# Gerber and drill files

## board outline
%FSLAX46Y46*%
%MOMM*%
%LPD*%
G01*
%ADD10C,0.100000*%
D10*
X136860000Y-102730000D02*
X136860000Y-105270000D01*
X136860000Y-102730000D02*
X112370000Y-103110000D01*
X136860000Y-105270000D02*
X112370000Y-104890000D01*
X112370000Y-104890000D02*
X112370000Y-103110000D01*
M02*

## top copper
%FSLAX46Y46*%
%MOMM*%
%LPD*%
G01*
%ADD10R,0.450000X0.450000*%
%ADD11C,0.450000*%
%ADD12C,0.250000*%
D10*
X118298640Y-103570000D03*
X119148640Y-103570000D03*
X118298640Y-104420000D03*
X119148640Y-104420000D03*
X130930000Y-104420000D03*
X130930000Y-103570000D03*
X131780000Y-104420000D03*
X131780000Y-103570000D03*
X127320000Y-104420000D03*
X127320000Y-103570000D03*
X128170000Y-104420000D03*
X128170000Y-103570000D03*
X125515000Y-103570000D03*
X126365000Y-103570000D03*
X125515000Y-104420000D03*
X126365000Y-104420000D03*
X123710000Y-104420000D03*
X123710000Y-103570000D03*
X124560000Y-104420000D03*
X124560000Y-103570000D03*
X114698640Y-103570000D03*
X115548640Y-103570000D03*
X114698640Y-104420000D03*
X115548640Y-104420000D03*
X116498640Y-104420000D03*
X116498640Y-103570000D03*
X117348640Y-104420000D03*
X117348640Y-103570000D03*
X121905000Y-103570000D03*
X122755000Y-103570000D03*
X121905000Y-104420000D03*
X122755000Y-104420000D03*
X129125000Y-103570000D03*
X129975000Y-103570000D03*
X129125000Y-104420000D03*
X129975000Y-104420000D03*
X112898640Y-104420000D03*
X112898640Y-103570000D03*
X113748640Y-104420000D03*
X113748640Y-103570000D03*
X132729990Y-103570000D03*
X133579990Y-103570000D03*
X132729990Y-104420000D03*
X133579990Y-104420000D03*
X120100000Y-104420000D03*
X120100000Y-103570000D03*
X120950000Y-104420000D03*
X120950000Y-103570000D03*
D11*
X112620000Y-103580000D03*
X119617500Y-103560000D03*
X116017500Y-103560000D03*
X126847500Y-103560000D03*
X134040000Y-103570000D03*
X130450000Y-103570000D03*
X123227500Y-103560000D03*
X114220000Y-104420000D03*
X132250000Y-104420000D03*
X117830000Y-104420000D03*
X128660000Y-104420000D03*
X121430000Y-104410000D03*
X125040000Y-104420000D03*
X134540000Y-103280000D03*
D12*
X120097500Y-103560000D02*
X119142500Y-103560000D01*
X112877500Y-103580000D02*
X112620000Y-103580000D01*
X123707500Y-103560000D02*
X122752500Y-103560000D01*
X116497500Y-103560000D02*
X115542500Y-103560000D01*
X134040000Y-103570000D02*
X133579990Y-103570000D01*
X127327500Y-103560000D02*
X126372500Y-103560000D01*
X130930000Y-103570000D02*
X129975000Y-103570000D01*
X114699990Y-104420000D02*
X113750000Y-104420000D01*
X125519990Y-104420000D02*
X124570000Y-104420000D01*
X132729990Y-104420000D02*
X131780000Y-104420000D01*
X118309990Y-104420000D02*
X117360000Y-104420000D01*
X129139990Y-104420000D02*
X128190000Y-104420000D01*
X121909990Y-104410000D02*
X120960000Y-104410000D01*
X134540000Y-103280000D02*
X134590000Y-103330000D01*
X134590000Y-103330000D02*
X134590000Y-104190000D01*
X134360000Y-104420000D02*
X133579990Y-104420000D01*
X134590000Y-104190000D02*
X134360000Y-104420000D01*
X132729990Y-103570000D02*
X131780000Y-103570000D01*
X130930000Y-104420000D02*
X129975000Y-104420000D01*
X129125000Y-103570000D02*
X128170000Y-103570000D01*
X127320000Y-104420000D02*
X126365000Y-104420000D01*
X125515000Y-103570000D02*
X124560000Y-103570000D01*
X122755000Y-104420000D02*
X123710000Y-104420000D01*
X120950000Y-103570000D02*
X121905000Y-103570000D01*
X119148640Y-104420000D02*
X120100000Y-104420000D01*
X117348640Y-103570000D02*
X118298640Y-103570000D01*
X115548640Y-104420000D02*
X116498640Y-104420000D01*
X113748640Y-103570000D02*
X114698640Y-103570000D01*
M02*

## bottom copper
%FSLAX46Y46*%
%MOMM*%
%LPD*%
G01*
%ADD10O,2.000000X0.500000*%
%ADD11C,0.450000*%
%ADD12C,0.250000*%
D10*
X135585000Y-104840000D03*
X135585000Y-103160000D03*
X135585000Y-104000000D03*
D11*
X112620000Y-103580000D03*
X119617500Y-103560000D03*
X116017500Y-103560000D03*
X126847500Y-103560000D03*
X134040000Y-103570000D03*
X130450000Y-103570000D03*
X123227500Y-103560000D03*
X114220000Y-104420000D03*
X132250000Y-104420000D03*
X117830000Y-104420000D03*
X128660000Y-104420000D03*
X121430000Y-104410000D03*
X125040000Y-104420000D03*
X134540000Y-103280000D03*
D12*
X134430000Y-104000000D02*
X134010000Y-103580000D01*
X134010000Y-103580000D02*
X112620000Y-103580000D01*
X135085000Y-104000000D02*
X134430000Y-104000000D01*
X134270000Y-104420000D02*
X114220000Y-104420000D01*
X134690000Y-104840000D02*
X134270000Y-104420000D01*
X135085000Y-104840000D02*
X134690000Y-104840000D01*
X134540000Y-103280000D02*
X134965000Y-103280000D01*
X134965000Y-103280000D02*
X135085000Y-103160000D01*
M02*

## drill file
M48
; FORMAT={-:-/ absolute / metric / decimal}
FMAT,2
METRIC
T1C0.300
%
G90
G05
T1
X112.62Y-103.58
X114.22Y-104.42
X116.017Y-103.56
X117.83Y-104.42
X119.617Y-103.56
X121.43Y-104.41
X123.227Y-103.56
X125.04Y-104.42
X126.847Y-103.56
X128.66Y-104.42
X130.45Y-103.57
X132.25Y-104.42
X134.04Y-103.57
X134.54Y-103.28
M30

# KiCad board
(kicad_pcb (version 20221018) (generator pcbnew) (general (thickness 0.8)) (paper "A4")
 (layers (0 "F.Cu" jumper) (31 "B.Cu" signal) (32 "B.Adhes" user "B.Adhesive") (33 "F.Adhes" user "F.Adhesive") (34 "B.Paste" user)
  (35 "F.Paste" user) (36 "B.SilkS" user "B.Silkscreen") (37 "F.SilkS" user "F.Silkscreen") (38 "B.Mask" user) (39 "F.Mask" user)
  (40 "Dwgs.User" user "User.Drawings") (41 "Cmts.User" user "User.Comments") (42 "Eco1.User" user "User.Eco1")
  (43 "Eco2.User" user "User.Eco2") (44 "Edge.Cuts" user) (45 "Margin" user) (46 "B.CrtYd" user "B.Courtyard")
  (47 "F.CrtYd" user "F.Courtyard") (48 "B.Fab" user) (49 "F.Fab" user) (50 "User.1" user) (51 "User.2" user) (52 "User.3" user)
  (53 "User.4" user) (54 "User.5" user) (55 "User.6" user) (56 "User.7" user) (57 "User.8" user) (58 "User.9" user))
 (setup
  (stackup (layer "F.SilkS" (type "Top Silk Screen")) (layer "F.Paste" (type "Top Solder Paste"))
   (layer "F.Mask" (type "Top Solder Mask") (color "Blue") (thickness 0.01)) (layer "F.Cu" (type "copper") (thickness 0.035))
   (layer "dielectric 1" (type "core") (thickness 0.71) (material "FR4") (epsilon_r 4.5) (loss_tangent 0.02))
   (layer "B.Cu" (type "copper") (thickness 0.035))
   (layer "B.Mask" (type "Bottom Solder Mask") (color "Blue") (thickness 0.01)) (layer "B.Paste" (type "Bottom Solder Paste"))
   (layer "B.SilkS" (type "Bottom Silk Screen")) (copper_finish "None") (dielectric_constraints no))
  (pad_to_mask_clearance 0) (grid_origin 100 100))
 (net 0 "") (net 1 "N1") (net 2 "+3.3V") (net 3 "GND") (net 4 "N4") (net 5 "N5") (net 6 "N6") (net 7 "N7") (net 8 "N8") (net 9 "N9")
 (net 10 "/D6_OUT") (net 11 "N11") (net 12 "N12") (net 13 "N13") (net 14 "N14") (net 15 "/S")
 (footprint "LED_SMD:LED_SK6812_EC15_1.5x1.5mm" (layer "F.Cu") (at 118.72364 103.995)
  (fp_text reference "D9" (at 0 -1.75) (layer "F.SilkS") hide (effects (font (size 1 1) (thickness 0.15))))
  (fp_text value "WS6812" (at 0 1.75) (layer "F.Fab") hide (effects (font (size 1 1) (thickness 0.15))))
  (pad "1" smd rect (at -0.425 -0.425) (size 0.45 0.45) (layers "F.Cu" "F.Paste" "F.Mask") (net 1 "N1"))
  (pad "2" smd rect (at 0.425 -0.425) (size 0.45 0.45) (layers "F.Cu" "F.Paste" "F.Mask") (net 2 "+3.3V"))
  (pad "3" smd rect (at -0.425 0.425) (size 0.45 0.45) (layers "F.Cu" "F.Paste" "F.Mask") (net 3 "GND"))
  (pad "4" smd rect (at 0.425 0.425) (size 0.45 0.45) (layers "F.Cu" "F.Paste" "F.Mask") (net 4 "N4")))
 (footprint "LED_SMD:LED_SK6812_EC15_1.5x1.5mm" (layer "F.Cu") (at 131.355 103.995 90)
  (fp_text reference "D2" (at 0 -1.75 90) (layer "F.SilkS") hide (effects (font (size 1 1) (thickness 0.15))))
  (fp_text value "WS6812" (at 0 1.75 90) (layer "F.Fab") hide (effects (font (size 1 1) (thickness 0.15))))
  (pad "1" smd rect (at -0.425 -0.425 90) (size 0.45 0.45) (layers "F.Cu" "F.Paste" "F.Mask") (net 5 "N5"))
  (pad "2" smd rect (at 0.425 -0.425 90) (size 0.45 0.45) (layers "F.Cu" "F.Paste" "F.Mask") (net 2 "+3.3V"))
  (pad "3" smd rect (at -0.425 0.425 90) (size 0.45 0.45) (layers "F.Cu" "F.Paste" "F.Mask") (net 3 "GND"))
  (pad "4" smd rect (at 0.425 0.425 90) (size 0.45 0.45) (layers "F.Cu" "F.Paste" "F.Mask") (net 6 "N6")))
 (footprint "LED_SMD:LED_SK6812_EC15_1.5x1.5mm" (layer "F.Cu") (at 127.745 103.995 90)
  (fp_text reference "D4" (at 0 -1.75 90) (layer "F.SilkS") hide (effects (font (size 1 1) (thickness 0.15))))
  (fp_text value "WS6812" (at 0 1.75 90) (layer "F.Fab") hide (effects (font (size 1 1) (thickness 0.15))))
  (pad "1" smd rect (at -0.425 -0.425 90) (size 0.45 0.45) (layers "F.Cu" "F.Paste" "F.Mask") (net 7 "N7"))
  (pad "2" smd rect (at 0.425 -0.425 90) (size 0.45 0.45) (layers "F.Cu" "F.Paste" "F.Mask") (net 2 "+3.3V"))
  (pad "3" smd rect (at -0.425 0.425 90) (size 0.45 0.45) (layers "F.Cu" "F.Paste" "F.Mask") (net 3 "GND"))
  (pad "4" smd rect (at 0.425 0.425 90) (size 0.45 0.45) (layers "F.Cu" "F.Paste" "F.Mask") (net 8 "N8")))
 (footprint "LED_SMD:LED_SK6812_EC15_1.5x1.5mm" (layer "F.Cu") (at 125.94 103.995)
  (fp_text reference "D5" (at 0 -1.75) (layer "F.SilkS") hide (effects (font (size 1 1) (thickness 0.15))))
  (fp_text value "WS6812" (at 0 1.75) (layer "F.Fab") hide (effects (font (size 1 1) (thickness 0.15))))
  (pad "1" smd rect (at -0.425 -0.425) (size 0.45 0.45) (layers "F.Cu" "F.Paste" "F.Mask") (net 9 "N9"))
  (pad "2" smd rect (at 0.425 -0.425) (size 0.45 0.45) (layers "F.Cu" "F.Paste" "F.Mask") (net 2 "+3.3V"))
  (pad "3" smd rect (at -0.425 0.425) (size 0.45 0.45) (layers "F.Cu" "F.Paste" "F.Mask") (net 3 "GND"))
  (pad "4" smd rect (at 0.425 0.425) (size 0.45 0.45) (layers "F.Cu" "F.Paste" "F.Mask") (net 7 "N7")))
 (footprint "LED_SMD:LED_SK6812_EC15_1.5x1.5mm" (layer "F.Cu") (at 124.135 103.995 90)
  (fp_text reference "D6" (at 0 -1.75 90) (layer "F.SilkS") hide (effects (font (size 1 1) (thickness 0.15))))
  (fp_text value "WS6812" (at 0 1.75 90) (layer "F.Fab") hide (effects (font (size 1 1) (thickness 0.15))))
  (pad "1" smd rect (at -0.425 -0.425 90) (size 0.45 0.45) (layers "F.Cu" "F.Paste" "F.Mask") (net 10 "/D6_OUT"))
  (pad "2" smd rect (at 0.425 -0.425 90) (size 0.45 0.45) (layers "F.Cu" "F.Paste" "F.Mask") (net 2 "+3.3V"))
  (pad "3" smd rect (at -0.425 0.425 90) (size 0.45 0.45) (layers "F.Cu" "F.Paste" "F.Mask") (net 3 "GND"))
  (pad "4" smd rect (at 0.425 0.425 90) (size 0.45 0.45) (layers "F.Cu" "F.Paste" "F.Mask") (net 9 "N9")))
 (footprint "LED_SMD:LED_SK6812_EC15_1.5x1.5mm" (layer "F.Cu") (at 115.12364 103.995)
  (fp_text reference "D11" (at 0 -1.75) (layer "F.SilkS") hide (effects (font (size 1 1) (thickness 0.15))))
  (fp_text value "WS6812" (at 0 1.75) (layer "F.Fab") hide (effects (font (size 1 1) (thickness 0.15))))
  (pad "1" smd rect (at -0.425 -0.425) (size 0.45 0.45) (layers "F.Cu" "F.Paste" "F.Mask") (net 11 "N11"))
  (pad "2" smd rect (at 0.425 -0.425) (size 0.45 0.45) (layers "F.Cu" "F.Paste" "F.Mask") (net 2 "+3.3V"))
  (pad "3" smd rect (at -0.425 0.425) (size 0.45 0.45) (layers "F.Cu" "F.Paste" "F.Mask") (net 3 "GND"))
  (pad "4" smd rect (at 0.425 0.425) (size 0.45 0.45) (layers "F.Cu" "F.Paste" "F.Mask") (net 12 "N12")))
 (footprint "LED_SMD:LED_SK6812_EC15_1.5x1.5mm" (layer "F.Cu") (at 116.92364 103.995 90)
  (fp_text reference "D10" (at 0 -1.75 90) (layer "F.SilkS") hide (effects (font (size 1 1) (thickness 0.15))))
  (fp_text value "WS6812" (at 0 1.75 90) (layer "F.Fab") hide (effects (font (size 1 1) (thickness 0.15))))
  (pad "1" smd rect (at -0.425 -0.425 90) (size 0.45 0.45) (layers "F.Cu" "F.Paste" "F.Mask") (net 12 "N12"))
  (pad "2" smd rect (at 0.425 -0.425 90) (size 0.45 0.45) (layers "F.Cu" "F.Paste" "F.Mask") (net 2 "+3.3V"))
  (pad "3" smd rect (at -0.425 0.425 90) (size 0.45 0.45) (layers "F.Cu" "F.Paste" "F.Mask") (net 3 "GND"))
  (pad "4" smd rect (at 0.425 0.425 90) (size 0.45 0.45) (layers "F.Cu" "F.Paste" "F.Mask") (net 1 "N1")))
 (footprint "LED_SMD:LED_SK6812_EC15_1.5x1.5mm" (layer "F.Cu") (at 122.33 103.995)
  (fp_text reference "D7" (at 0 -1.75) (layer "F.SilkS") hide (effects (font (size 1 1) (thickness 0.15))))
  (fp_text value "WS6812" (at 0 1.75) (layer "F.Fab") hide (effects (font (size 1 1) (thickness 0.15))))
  (pad "1" smd rect (at -0.425 -0.425) (size 0.45 0.45) (layers "F.Cu" "F.Paste" "F.Mask") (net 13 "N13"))
  (pad "2" smd rect (at 0.425 -0.425) (size 0.45 0.45) (layers "F.Cu" "F.Paste" "F.Mask") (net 2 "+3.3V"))
  (pad "3" smd rect (at -0.425 0.425) (size 0.45 0.45) (layers "F.Cu" "F.Paste" "F.Mask") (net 3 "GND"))
  (pad "4" smd rect (at 0.425 0.425) (size 0.45 0.45) (layers "F.Cu" "F.Paste" "F.Mask") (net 10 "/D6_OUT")))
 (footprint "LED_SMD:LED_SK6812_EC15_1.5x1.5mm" (layer "F.Cu") (at 129.55 103.995)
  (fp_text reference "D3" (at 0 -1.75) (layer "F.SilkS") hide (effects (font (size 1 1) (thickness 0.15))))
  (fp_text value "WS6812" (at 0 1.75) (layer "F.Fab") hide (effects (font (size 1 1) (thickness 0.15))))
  (pad "1" smd rect (at -0.425 -0.425) (size 0.45 0.45) (layers "F.Cu" "F.Paste" "F.Mask") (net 8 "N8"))
  (pad "2" smd rect (at 0.425 -0.425) (size 0.45 0.45) (layers "F.Cu" "F.Paste" "F.Mask") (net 2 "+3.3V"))
  (pad "3" smd rect (at -0.425 0.425) (size 0.45 0.45) (layers "F.Cu" "F.Paste" "F.Mask") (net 3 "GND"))
  (pad "4" smd rect (at 0.425 0.425) (size 0.45 0.45) (layers "F.Cu" "F.Paste" "F.Mask") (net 5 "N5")))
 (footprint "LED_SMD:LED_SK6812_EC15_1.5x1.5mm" (layer "F.Cu") (at 113.32364 103.995 90)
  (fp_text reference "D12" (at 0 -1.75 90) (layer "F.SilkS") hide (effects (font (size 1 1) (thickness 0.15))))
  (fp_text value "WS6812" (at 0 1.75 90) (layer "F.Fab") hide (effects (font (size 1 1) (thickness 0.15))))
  (pad "1" smd rect (at -0.425 -0.425 90) (size 0.45 0.45) (layers "F.Cu" "F.Paste" "F.Mask") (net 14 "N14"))
  (pad "2" smd rect (at 0.425 -0.425 90) (size 0.45 0.45) (layers "F.Cu" "F.Paste" "F.Mask") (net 2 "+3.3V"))
  (pad "3" smd rect (at -0.425 0.425 90) (size 0.45 0.45) (layers "F.Cu" "F.Paste" "F.Mask") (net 3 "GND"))
  (pad "4" smd rect (at 0.425 0.425 90) (size 0.45 0.45) (layers "F.Cu" "F.Paste" "F.Mask") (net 11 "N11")))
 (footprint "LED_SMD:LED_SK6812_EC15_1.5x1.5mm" (layer "F.Cu") (at 133.15499 103.995)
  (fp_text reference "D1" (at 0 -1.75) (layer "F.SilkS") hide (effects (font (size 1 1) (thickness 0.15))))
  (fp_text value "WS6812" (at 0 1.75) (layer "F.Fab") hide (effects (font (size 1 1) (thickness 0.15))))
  (pad "1" smd rect (at -0.425 -0.425) (size 0.45 0.45) (layers "F.Cu" "F.Paste" "F.Mask") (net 6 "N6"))
  (pad "2" smd rect (at 0.425 -0.425) (size 0.45 0.45) (layers "F.Cu" "F.Paste" "F.Mask") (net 2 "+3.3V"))
  (pad "3" smd rect (at -0.425 0.425) (size 0.45 0.45) (layers "F.Cu" "F.Paste" "F.Mask") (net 3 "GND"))
  (pad "4" smd rect (at 0.425 0.425) (size 0.45 0.45) (layers "F.Cu" "F.Paste" "F.Mask") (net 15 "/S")))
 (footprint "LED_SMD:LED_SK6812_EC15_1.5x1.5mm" (layer "F.Cu") (at 120.525 103.995 90)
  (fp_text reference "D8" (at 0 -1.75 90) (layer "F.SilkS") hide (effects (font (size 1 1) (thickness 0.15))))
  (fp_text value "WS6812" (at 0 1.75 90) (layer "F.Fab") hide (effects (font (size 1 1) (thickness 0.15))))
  (pad "1" smd rect (at -0.425 -0.425 90) (size 0.45 0.45) (layers "F.Cu" "F.Paste" "F.Mask") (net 4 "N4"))
  (pad "2" smd rect (at 0.425 -0.425 90) (size 0.45 0.45) (layers "F.Cu" "F.Paste" "F.Mask") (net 2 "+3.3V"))
  (pad "3" smd rect (at -0.425 0.425 90) (size 0.45 0.45) (layers "F.Cu" "F.Paste" "F.Mask") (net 3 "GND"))
  (pad "4" smd rect (at 0.425 0.425 90) (size 0.45 0.45) (layers "F.Cu" "F.Paste" "F.Mask") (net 13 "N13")))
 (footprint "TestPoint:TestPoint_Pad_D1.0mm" (layer "B.Cu") (at 135.585 104.84 180)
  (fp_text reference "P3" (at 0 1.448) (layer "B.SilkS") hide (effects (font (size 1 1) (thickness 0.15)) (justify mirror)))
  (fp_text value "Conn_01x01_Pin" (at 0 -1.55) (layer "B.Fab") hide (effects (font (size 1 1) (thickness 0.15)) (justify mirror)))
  (pad "1" smd oval (at 0 0 180) (size 2 0.5) (layers "B.Cu" "B.Mask") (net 3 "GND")))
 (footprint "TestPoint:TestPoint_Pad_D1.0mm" (layer "B.Cu") (at 135.585 103.16 180)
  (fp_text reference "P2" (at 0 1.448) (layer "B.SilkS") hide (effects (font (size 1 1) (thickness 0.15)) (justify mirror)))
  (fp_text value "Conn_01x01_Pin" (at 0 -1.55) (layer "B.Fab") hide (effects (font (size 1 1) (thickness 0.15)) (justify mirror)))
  (pad "1" smd oval (at 0 0 180) (size 2 0.5) (layers "B.Cu" "B.Mask") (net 15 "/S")))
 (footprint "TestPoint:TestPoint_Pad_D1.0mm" (layer "B.Cu") (at 135.585 104 180)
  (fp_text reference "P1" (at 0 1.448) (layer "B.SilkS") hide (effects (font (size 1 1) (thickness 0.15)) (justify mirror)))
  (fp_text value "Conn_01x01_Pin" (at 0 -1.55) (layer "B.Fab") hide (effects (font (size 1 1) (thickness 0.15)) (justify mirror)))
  (pad "1" smd oval (at 0 0 180) (size 2 0.5) (layers "B.Cu" "B.Mask") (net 2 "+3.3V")))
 (gr_line (start 136.86 102.73) (end 136.86 105.27) (stroke (width 0.1) (type default)) (layer "Edge.Cuts"))
 (gr_line (start 136.86 102.73) (end 112.37 103.11) (stroke (width 0.1) (type default)) (layer "Edge.Cuts"))
 (gr_line (start 136.86 105.27) (end 112.37 104.89) (stroke (width 0.1) (type default)) (layer "Edge.Cuts"))
 (gr_line (start 112.37 104.89) (end 112.37 103.11) (stroke (width 0.1) (type default)) (layer "Edge.Cuts"))
 (segment (start 120.0975 103.56) (end 119.1425 103.56) (width 0.25) (layer "F.Cu") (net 2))
 (segment (start 112.8775 103.58) (end 112.62 103.58) (width 0.25) (layer "F.Cu") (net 2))
 (segment (start 123.7075 103.56) (end 122.7525 103.56) (width 0.25) (layer "F.Cu") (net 2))
 (segment (start 116.4975 103.56) (end 115.5425 103.56) (width 0.25) (layer "F.Cu") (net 2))
 (segment (start 134.04 103.57) (end 133.57999 103.57) (width 0.25) (layer "F.Cu") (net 2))
 (segment (start 127.3275 103.56) (end 126.3725 103.56) (width 0.25) (layer "F.Cu") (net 2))
 (segment (start 130.93 103.57) (end 129.975 103.57) (width 0.25) (layer "F.Cu") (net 2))
 (via (at 112.62 103.58) (size 0.45) (drill 0.3) (layers "F.Cu" "B.Cu") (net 2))
 (via (at 119.6175 103.56) (size 0.45) (drill 0.3) (layers "F.Cu" "B.Cu") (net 2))
 (via (at 116.0175 103.56) (size 0.45) (drill 0.3) (layers "F.Cu" "B.Cu") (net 2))
 (via (at 126.8475 103.56) (size 0.45) (drill 0.3) (layers "F.Cu" "B.Cu") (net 2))
 (via (at 134.04 103.57) (size 0.45) (drill 0.3) (layers "F.Cu" "B.Cu") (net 2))
 (via (at 130.45 103.57) (size 0.45) (drill 0.3) (layers "F.Cu" "B.Cu") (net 2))
 (via (at 123.2275 103.56) (size 0.45) (drill 0.3) (layers "F.Cu" "B.Cu") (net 2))
 (segment (start 134.43 104) (end 134.01 103.58) (width 0.25) (layer "B.Cu") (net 2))
 (segment (start 134.01 103.58) (end 112.62 103.58) (width 0.25) (layer "B.Cu") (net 2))
 (segment (start 135.085 104) (end 134.43 104) (width 0.25) (layer "B.Cu") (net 2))
 (segment (start 114.69999 104.42) (end 113.75 104.42) (width 0.25) (layer "F.Cu") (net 3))
 (segment (start 125.51999 104.42) (end 124.57 104.42) (width 0.25) (layer "F.Cu") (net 3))
 (segment (start 132.72999 104.42) (end 131.78 104.42) (width 0.25) (layer "F.Cu") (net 3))
 (segment (start 118.30999 104.42) (end 117.36 104.42) (width 0.25) (layer "F.Cu") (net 3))
 (segment (start 129.13999 104.42) (end 128.19 104.42) (width 0.25) (layer "F.Cu") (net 3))
 (segment (start 121.90999 104.41) (end 120.96 104.41) (width 0.25) (layer "F.Cu") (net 3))
 (via (at 114.22 104.42) (size 0.45) (drill 0.3) (layers "F.Cu" "B.Cu") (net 3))
 (via (at 132.25 104.42) (size 0.45) (drill 0.3) (layers "F.Cu" "B.Cu") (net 3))
 (via (at 117.83 104.42) (size 0.45) (drill 0.3) (layers "F.Cu" "B.Cu") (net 3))
 (via (at 128.66 104.42) (size 0.45) (drill 0.3) (layers "F.Cu" "B.Cu") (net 3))
 (via (at 121.43 104.41) (size 0.45) (drill 0.3) (layers "F.Cu" "B.Cu") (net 3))
 (via (at 125.04 104.42) (size 0.45) (drill 0.3) (layers "F.Cu" "B.Cu") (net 3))
 (segment (start 134.27 104.42) (end 114.22 104.42) (width 0.25) (layer "B.Cu") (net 3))
 (segment (start 134.69 104.84) (end 134.27 104.42) (width 0.25) (layer "B.Cu") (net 3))
 (segment (start 135.085 104.84) (end 134.69 104.84) (width 0.25) (layer "B.Cu") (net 3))
 (segment (start 134.54 103.28) (end 134.59 103.33) (width 0.25) (layer "F.Cu") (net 15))
 (segment (start 134.59 103.33) (end 134.59 104.19) (width 0.25) (layer "F.Cu") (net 15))
 (segment (start 134.36 104.42) (end 133.57999 104.42) (width 0.25) (layer "F.Cu") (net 15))
 (segment (start 134.59 104.19) (end 134.36 104.42) (width 0.25) (layer "F.Cu") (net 15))
 (via (at 134.54 103.28) (size 0.45) (drill 0.3) (layers "F.Cu" "B.Cu") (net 15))
 (segment (start 134.54 103.28) (end 134.965 103.28) (width 0.25) (layer "B.Cu") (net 15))
 (segment (start 134.965 103.28) (end 135.085 103.16) (width 0.25) (layer "B.Cu") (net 15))
 (segment (start 132.72999 103.57) (end 131.78 103.57) (width 0.25) (layer "F.Cu") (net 6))
 (segment (start 130.93 104.42) (end 129.975 104.42) (width 0.25) (layer "F.Cu") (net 5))
 (segment (start 129.125 103.57) (end 128.17 103.57) (width 0.25) (layer "F.Cu") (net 8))
 (segment (start 127.32 104.42) (end 126.365 104.42) (width 0.25) (layer "F.Cu") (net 7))
 (segment (start 125.515 103.57) (end 124.56 103.57) (width 0.25) (layer "F.Cu") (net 9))
 (segment (start 122.755 104.42) (end 123.71 104.42) (width 0.25) (layer "F.Cu") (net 10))
 (segment (start 120.95 103.57) (end 121.905 103.57) (width 0.25) (layer "F.Cu") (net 13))
 (segment (start 119.14864 104.42) (end 120.1 104.42) (width 0.25) (layer "F.Cu") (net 4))
 (segment (start 117.34864 103.57) (end 118.29864 103.57) (width 0.25) (layer "F.Cu") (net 1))
 (segment (start 115.54864 104.42) (end 116.49864 104.42) (width 0.25) (layer "F.Cu") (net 12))
 (segment (start 113.74864 103.57) (end 114.69864 103.57) (width 0.25) (layer "F.Cu") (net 11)))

